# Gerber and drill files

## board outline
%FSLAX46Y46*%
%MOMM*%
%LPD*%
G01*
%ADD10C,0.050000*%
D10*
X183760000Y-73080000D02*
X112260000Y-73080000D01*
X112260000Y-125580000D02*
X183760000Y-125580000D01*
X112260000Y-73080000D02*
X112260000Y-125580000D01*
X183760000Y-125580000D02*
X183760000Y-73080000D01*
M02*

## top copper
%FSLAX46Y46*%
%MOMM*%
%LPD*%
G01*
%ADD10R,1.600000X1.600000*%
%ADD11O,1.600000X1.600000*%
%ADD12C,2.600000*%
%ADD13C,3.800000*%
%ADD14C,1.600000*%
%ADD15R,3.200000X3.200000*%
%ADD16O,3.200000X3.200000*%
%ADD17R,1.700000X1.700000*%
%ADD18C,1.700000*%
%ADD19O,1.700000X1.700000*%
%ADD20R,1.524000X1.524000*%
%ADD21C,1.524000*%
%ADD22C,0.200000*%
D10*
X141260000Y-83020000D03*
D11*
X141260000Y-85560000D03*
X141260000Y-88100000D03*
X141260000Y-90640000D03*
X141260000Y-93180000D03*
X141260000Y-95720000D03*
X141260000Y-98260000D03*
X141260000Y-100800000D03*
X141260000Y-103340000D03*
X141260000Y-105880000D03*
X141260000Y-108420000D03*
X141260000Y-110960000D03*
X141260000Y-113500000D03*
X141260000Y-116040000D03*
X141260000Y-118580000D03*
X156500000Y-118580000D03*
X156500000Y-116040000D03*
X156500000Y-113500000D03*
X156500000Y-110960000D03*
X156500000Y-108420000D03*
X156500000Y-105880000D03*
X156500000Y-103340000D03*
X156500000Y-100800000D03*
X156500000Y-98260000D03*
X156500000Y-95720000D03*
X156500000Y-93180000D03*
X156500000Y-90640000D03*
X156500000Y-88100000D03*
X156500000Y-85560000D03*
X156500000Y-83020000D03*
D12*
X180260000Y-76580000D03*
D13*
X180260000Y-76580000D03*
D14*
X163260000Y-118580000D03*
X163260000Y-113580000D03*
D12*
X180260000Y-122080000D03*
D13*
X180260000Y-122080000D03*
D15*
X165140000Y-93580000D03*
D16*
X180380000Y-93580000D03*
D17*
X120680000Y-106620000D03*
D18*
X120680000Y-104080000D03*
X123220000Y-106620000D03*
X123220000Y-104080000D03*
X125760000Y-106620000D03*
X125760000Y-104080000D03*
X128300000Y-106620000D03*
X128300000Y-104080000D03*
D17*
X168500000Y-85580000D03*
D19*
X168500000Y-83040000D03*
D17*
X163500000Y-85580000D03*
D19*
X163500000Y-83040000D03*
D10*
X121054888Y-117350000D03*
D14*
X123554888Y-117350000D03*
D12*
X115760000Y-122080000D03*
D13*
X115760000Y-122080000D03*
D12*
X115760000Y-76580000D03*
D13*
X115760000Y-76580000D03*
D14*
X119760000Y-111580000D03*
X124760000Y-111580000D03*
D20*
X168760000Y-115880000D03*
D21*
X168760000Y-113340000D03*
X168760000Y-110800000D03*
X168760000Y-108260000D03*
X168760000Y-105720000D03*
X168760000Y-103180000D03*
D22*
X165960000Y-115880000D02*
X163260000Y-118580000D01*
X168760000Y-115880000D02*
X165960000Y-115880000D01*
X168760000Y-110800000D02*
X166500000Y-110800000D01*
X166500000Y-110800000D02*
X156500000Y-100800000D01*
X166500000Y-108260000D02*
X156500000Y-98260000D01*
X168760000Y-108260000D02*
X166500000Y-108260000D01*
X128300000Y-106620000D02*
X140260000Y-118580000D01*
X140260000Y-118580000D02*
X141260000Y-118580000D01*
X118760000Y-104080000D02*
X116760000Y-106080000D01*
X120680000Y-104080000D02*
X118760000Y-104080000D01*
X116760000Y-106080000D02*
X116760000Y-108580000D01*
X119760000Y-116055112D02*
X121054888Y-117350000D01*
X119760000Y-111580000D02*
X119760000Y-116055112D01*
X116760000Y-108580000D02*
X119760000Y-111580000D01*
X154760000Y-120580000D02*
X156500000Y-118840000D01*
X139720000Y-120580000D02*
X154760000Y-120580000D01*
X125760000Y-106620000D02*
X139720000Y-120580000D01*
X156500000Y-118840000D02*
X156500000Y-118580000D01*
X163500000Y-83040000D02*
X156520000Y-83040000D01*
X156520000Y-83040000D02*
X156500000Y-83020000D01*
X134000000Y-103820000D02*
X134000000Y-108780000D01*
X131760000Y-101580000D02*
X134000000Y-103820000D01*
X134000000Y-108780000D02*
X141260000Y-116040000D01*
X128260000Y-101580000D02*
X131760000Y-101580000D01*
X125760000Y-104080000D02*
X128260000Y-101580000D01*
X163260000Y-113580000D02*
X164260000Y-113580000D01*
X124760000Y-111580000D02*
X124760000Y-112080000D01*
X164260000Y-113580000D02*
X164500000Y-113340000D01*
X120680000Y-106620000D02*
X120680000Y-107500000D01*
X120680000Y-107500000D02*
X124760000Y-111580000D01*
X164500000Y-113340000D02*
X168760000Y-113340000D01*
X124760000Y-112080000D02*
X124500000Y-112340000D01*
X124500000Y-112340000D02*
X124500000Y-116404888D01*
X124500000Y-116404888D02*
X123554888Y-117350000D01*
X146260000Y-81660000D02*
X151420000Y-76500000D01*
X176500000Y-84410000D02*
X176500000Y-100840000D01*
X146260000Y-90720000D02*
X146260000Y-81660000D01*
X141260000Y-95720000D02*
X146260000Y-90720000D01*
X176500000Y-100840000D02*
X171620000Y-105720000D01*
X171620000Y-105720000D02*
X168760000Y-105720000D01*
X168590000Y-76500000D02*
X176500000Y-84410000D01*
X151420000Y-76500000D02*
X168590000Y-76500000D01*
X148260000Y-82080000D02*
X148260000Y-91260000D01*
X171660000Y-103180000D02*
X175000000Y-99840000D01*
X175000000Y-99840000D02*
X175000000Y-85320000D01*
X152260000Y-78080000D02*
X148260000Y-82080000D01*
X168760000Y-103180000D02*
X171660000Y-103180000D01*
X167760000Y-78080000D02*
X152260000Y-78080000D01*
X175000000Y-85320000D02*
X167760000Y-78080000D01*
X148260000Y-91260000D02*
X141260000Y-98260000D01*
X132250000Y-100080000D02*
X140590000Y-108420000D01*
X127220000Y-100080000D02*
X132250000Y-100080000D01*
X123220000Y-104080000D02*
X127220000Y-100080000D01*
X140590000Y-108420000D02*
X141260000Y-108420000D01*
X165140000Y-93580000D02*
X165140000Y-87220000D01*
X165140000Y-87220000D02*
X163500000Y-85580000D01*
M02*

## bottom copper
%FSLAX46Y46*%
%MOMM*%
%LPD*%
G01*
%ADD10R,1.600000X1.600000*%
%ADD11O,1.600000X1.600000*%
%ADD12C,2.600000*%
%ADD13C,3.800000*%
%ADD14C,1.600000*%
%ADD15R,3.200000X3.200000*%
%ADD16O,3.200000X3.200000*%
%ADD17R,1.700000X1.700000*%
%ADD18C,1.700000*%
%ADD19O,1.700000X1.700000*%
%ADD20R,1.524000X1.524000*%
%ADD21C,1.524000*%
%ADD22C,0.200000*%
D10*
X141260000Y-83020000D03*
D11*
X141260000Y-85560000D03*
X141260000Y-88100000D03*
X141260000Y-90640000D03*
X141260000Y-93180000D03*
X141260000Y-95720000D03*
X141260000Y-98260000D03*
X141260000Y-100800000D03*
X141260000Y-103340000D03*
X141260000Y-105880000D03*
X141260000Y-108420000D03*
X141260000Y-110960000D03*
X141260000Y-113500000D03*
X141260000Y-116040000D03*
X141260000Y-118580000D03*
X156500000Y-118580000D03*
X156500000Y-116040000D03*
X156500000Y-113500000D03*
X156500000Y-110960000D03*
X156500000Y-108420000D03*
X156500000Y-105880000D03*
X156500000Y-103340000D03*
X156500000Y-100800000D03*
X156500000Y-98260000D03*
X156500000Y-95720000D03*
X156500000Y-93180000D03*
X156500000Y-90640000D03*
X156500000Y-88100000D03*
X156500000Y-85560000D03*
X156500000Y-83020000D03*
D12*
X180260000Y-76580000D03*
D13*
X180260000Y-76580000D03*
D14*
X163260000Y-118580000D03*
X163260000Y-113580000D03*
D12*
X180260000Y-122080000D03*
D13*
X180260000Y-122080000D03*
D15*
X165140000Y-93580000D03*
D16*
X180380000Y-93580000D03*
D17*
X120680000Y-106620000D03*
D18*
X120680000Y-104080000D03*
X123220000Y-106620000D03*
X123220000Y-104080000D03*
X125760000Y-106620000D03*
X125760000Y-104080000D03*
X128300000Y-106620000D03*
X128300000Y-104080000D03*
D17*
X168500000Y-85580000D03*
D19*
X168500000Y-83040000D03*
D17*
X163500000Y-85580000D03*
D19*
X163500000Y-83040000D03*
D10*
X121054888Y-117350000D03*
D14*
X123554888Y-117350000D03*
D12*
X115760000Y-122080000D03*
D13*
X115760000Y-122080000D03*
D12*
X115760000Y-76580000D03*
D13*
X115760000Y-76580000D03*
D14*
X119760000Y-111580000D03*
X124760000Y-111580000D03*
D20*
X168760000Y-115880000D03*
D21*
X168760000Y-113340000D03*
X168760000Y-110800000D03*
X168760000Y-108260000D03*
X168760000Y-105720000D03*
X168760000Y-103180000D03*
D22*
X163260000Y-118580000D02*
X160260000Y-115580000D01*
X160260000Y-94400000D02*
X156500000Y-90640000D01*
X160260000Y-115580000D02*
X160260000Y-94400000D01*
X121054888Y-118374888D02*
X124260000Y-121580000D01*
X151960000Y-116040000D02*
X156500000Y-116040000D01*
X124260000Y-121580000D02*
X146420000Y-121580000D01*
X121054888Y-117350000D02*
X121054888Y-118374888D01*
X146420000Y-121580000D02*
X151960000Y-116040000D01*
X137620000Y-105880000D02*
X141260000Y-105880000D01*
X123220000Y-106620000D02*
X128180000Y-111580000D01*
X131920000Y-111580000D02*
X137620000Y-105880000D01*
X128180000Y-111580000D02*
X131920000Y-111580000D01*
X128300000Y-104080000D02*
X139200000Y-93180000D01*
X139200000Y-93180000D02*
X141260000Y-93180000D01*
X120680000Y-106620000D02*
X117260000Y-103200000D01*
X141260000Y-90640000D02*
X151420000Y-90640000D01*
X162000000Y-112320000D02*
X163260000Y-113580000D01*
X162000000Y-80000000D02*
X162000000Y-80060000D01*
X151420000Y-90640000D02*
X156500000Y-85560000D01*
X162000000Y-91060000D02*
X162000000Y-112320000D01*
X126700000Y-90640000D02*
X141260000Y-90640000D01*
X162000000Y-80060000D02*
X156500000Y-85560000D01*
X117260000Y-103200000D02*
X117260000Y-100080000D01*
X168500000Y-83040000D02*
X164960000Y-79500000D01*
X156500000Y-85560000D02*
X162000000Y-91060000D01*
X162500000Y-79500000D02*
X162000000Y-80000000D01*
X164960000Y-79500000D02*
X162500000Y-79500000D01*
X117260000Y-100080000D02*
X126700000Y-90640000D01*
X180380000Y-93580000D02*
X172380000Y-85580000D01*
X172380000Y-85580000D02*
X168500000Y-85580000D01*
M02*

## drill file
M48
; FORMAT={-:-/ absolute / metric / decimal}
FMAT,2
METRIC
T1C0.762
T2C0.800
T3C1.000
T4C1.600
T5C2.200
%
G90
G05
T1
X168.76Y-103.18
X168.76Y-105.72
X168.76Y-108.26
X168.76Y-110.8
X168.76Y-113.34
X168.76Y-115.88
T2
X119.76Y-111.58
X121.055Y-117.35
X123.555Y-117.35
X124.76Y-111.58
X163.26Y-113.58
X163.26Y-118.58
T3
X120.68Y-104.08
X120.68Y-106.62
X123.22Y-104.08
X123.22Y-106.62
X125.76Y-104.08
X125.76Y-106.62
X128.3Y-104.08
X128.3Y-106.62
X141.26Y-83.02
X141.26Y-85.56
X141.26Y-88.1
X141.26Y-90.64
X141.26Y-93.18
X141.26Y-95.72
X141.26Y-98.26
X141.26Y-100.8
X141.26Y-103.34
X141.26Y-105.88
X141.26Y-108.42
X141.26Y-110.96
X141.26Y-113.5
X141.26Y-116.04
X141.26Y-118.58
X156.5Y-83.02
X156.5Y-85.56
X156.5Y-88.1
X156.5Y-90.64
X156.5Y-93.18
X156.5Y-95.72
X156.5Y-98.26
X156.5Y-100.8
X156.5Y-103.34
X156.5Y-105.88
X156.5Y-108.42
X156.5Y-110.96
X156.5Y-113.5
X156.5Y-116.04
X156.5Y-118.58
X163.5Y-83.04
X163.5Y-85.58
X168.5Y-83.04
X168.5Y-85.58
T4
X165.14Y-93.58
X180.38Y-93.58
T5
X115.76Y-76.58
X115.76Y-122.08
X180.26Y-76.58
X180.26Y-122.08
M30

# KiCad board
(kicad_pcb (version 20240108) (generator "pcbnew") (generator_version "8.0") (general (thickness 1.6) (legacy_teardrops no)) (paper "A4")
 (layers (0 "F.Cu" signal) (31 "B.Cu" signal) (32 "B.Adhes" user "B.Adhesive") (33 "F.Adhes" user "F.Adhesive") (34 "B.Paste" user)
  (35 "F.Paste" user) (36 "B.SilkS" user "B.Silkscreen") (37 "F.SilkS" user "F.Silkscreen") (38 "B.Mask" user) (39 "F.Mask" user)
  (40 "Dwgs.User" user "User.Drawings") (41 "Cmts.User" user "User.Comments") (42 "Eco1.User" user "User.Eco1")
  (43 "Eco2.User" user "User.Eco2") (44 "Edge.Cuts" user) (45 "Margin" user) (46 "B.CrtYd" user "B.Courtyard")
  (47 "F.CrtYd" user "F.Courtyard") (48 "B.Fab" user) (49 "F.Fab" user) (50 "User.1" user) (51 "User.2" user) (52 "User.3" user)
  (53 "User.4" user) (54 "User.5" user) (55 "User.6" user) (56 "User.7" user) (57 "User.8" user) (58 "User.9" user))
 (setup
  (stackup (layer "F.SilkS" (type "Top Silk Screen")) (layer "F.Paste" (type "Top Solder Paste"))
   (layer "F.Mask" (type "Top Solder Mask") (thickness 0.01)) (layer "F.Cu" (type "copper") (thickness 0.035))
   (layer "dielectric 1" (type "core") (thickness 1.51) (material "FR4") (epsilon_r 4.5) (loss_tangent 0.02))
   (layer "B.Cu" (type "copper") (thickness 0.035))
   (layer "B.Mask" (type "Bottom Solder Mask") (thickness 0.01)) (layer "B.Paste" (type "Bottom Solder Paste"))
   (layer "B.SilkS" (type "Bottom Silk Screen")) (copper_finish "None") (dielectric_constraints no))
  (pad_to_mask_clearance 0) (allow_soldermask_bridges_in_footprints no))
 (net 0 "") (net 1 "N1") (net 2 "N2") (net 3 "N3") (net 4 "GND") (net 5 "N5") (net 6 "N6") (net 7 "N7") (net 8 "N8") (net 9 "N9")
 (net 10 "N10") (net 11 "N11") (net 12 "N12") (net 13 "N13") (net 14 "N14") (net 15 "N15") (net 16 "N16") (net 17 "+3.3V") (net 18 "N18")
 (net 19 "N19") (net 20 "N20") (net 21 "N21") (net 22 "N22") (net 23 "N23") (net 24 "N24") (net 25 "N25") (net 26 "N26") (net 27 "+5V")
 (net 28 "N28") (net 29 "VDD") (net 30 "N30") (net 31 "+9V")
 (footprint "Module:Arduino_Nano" (layer "F.Cu") (at 141.26 83.02)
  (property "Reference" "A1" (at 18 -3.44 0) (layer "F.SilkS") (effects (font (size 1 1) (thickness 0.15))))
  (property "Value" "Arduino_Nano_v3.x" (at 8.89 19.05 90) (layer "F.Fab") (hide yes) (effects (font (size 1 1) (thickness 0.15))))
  (pad "1" thru_hole rect (at 0 0) (size 1.6 1.6) (drill 1) (layers "*.Cu" "*.Mask") (remove_unused_layers no) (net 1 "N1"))
  (pad "2" thru_hole oval (at 0 2.54) (size 1.6 1.6) (drill 1) (layers "*.Cu" "*.Mask") (remove_unused_layers no) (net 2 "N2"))
  (pad "3" thru_hole oval (at 0 5.08) (size 1.6 1.6) (drill 1) (layers "*.Cu" "*.Mask") (remove_unused_layers no) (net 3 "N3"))
  (pad "4" thru_hole oval (at 0 7.62) (size 1.6 1.6) (drill 1) (layers "*.Cu" "*.Mask") (remove_unused_layers no) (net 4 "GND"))
  (pad "5" thru_hole oval (at 0 10.16) (size 1.6 1.6) (drill 1) (layers "*.Cu" "*.Mask") (remove_unused_layers no) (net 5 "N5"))
  (pad "6" thru_hole oval (at 0 12.7) (size 1.6 1.6) (drill 1) (layers "*.Cu" "*.Mask") (remove_unused_layers no) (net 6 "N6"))
  (pad "7" thru_hole oval (at 0 15.24) (size 1.6 1.6) (drill 1) (layers "*.Cu" "*.Mask") (remove_unused_layers no) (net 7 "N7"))
  (pad "8" thru_hole oval (at 0 17.78) (size 1.6 1.6) (drill 1) (layers "*.Cu" "*.Mask") (remove_unused_layers no) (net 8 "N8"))
  (pad "9" thru_hole oval (at 0 20.32) (size 1.6 1.6) (drill 1) (layers "*.Cu" "*.Mask") (remove_unused_layers no) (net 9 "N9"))
  (pad "10" thru_hole oval (at 0 22.86) (size 1.6 1.6) (drill 1) (layers "*.Cu" "*.Mask") (remove_unused_layers no) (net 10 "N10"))
  (pad "11" thru_hole oval (at 0 25.4) (size 1.6 1.6) (drill 1) (layers "*.Cu" "*.Mask") (remove_unused_layers no) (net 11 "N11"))
  (pad "12" thru_hole oval (at 0 27.94) (size 1.6 1.6) (drill 1) (layers "*.Cu" "*.Mask") (remove_unused_layers no) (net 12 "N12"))
  (pad "13" thru_hole oval (at 0 30.48) (size 1.6 1.6) (drill 1) (layers "*.Cu" "*.Mask") (remove_unused_layers no) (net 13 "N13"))
  (pad "14" thru_hole oval (at 0 33.02) (size 1.6 1.6) (drill 1) (layers "*.Cu" "*.Mask") (remove_unused_layers no) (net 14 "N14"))
  (pad "15" thru_hole oval (at 0 35.56) (size 1.6 1.6) (drill 1) (layers "*.Cu" "*.Mask") (remove_unused_layers no) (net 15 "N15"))
  (pad "16" thru_hole oval (at 15.24 35.56) (size 1.6 1.6) (drill 1) (layers "*.Cu" "*.Mask") (remove_unused_layers no) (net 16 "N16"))
  (pad "17" thru_hole oval (at 15.24 33.02) (size 1.6 1.6) (drill 1) (layers "*.Cu" "*.Mask") (remove_unused_layers no) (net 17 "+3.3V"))
  (pad "18" thru_hole oval (at 15.24 30.48) (size 1.6 1.6) (drill 1) (layers "*.Cu" "*.Mask") (remove_unused_layers no) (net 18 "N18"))
  (pad "19" thru_hole oval (at 15.24 27.94) (size 1.6 1.6) (drill 1) (layers "*.Cu" "*.Mask") (remove_unused_layers no) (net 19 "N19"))
  (pad "20" thru_hole oval (at 15.24 25.4) (size 1.6 1.6) (drill 1) (layers "*.Cu" "*.Mask") (remove_unused_layers no) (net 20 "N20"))
  (pad "21" thru_hole oval (at 15.24 22.86) (size 1.6 1.6) (drill 1) (layers "*.Cu" "*.Mask") (remove_unused_layers no) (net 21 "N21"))
  (pad "22" thru_hole oval (at 15.24 20.32) (size 1.6 1.6) (drill 1) (layers "*.Cu" "*.Mask") (remove_unused_layers no) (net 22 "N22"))
  (pad "23" thru_hole oval (at 15.24 17.78) (size 1.6 1.6) (drill 1) (layers "*.Cu" "*.Mask") (remove_unused_layers no) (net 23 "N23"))
  (pad "24" thru_hole oval (at 15.24 15.24) (size 1.6 1.6) (drill 1) (layers "*.Cu" "*.Mask") (remove_unused_layers no) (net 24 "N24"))
  (pad "25" thru_hole oval (at 15.24 12.7) (size 1.6 1.6) (drill 1) (layers "*.Cu" "*.Mask") (remove_unused_layers no) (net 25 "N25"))
  (pad "26" thru_hole oval (at 15.24 10.16) (size 1.6 1.6) (drill 1) (layers "*.Cu" "*.Mask") (remove_unused_layers no) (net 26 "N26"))
  (pad "27" thru_hole oval (at 15.24 7.62) (size 1.6 1.6) (drill 1) (layers "*.Cu" "*.Mask") (remove_unused_layers no) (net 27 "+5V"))
  (pad "28" thru_hole oval (at 15.24 5.08) (size 1.6 1.6) (drill 1) (layers "*.Cu" "*.Mask") (remove_unused_layers no) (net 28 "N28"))
  (pad "29" thru_hole oval (at 15.24 2.54) (size 1.6 1.6) (drill 1) (layers "*.Cu" "*.Mask") (remove_unused_layers no) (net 4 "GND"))
  (pad "30" thru_hole oval (at 15.24 0) (size 1.6 1.6) (drill 1) (layers "*.Cu" "*.Mask") (remove_unused_layers no) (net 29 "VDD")))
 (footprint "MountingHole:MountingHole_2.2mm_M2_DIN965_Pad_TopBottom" (layer "F.Cu") (at 180.26 76.58)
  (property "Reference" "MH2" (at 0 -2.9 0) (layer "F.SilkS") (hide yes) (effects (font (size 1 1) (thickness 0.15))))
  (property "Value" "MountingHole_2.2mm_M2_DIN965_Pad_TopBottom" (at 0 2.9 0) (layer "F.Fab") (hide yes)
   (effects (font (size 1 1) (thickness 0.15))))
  (pad "1" thru_hole circle (at 0 0) (size 2.6 2.6) (drill 2.2) (layers "*.Cu" "*.Mask") (remove_unused_layers no))
  (pad "1" connect circle (at 0 0) (size 3.8 3.8) (layers "F.Cu" "F.Mask"))
  (pad "1" connect circle (at 0 0) (size 3.8 3.8) (layers "B.Cu" "B.Mask")))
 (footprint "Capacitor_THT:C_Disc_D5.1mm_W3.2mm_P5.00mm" (layer "F.Cu") (at 163.26 118.58 90)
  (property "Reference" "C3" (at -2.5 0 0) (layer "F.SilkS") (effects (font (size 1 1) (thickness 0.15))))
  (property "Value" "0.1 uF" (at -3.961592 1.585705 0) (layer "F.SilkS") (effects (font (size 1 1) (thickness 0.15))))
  (pad "1" thru_hole circle (at 0 0 90) (size 1.6 1.6) (drill 0.8) (layers "*.Cu" "*.Mask") (remove_unused_layers no) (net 27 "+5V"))
  (pad "2" thru_hole circle (at 5 0 90) (size 1.6 1.6) (drill 0.8) (layers "*.Cu" "*.Mask") (remove_unused_layers no) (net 4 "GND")))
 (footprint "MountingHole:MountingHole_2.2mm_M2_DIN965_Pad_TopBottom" (layer "F.Cu") (at 180.26 122.08)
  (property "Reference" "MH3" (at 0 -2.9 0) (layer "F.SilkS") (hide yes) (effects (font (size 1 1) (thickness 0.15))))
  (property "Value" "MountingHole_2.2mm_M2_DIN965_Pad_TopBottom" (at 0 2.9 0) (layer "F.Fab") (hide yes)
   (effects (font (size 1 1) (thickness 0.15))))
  (pad "1" thru_hole circle (at 0 0) (size 2.6 2.6) (drill 2.2) (layers "*.Cu" "*.Mask") (remove_unused_layers no))
  (pad "1" connect circle (at 0 0) (size 3.8 3.8) (layers "F.Cu" "F.Mask"))
  (pad "1" connect circle (at 0 0) (size 3.8 3.8) (layers "B.Cu" "B.Mask")))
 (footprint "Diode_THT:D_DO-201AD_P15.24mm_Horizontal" (layer "F.Cu") (at 165.14 93.58)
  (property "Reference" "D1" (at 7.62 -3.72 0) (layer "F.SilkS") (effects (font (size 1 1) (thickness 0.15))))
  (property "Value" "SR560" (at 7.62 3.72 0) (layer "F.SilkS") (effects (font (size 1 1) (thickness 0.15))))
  (pad "1" thru_hole rect (at 0 0) (size 3.2 3.2) (drill 1.6) (layers "*.Cu" "*.Mask") (remove_unused_layers no) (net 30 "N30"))
  (pad "2" thru_hole oval (at 15.24 0) (size 3.2 3.2) (drill 1.6) (layers "*.Cu" "*.Mask") (remove_unused_layers no) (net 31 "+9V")))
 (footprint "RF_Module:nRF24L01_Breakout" (layer "F.Cu") (at 120.68 106.62 90)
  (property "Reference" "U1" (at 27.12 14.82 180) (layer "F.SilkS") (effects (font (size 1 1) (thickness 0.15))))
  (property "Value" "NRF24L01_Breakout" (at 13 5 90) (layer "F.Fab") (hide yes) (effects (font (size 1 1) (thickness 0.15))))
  (pad "1" thru_hole rect (at 0 0 90) (size 1.7 1.7) (drill 1) (layers "*.Cu" "*.Mask") (remove_unused_layers no) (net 4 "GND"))
  (pad "2" thru_hole circle (at 2.54 0 90) (size 1.7 1.7) (drill 1) (layers "*.Cu" "*.Mask") (remove_unused_layers no) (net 17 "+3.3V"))
  (pad "3" thru_hole circle (at 0 2.54 90) (size 1.7 1.7) (drill 1) (layers "*.Cu" "*.Mask") (remove_unused_layers no) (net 10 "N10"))
  (pad "4" thru_hole circle (at 2.54 2.54 90) (size 1.7 1.7) (drill 1) (layers "*.Cu" "*.Mask") (remove_unused_layers no) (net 11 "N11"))
  (pad "5" thru_hole circle (at 0 5.08 90) (size 1.7 1.7) (drill 1) (layers "*.Cu" "*.Mask") (remove_unused_layers no) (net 16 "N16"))
  (pad "6" thru_hole circle (at 2.54 5.08 90) (size 1.7 1.7) (drill 1) (layers "*.Cu" "*.Mask") (remove_unused_layers no) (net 14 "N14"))
  (pad "7" thru_hole circle (at 0 7.62 90) (size 1.7 1.7) (drill 1) (layers "*.Cu" "*.Mask") (remove_unused_layers no) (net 15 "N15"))
  (pad "8" thru_hole circle (at 2.54 7.62 90) (size 1.7 1.7) (drill 1) (layers "*.Cu" "*.Mask") (remove_unused_layers no) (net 5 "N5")))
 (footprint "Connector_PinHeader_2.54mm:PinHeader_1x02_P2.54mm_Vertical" (layer "F.Cu") (at 168.5 85.58 180)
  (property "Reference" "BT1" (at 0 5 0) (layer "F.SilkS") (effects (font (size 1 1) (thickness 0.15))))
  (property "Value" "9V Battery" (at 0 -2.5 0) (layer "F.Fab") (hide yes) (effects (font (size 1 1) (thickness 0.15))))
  (pad "1" thru_hole rect (at 0 0 180) (size 1.7 1.7) (drill 1) (layers "*.Cu" "*.Mask") (remove_unused_layers no) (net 31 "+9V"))
  (pad "2" thru_hole oval (at 0 2.54 180) (size 1.7 1.7) (drill 1) (layers "*.Cu" "*.Mask") (remove_unused_layers no) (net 4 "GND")))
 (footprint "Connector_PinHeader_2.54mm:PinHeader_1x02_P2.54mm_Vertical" (layer "F.Cu") (at 163.5 85.58 180)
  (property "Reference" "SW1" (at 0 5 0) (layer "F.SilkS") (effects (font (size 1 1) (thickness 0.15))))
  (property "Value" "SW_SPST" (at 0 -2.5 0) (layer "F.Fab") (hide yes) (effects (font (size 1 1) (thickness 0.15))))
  (pad "1" thru_hole rect (at 0 0 180) (size 1.7 1.7) (drill 1) (layers "*.Cu" "*.Mask") (remove_unused_layers no) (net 30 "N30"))
  (pad "2" thru_hole oval (at 0 2.54 180) (size 1.7 1.7) (drill 1) (layers "*.Cu" "*.Mask") (remove_unused_layers no) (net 29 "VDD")))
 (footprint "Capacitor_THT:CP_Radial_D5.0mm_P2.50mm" (layer "F.Cu") (at 121.054888 117.35)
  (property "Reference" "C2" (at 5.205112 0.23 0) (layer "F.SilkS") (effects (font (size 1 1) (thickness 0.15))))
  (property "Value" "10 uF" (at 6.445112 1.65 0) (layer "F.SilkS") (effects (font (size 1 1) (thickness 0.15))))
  (pad "1" thru_hole rect (at 0 0) (size 1.6 1.6) (drill 0.8) (layers "*.Cu" "*.Mask") (remove_unused_layers no) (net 17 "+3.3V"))
  (pad "2" thru_hole circle (at 2.5 0) (size 1.6 1.6) (drill 0.8) (layers "*.Cu" "*.Mask") (remove_unused_layers no) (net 4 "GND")))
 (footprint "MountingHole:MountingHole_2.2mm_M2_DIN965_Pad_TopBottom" (layer "F.Cu") (at 115.76 122.08)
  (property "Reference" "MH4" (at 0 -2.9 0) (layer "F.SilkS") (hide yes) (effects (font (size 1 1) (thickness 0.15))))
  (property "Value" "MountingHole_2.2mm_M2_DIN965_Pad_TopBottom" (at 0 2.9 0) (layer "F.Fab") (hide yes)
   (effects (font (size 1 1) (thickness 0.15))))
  (pad "1" thru_hole circle (at 0 0) (size 2.6 2.6) (drill 2.2) (layers "*.Cu" "*.Mask") (remove_unused_layers no))
  (pad "1" connect circle (at 0 0) (size 3.8 3.8) (layers "F.Cu" "F.Mask"))
  (pad "1" connect circle (at 0 0) (size 3.8 3.8) (layers "B.Cu" "B.Mask")))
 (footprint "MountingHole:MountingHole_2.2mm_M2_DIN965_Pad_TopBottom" (layer "F.Cu") (at 115.76 76.58)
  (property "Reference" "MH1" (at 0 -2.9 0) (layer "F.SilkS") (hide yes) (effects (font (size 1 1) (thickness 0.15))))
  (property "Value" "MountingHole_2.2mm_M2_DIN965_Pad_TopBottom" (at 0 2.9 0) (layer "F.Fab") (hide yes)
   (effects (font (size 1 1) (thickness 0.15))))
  (pad "1" thru_hole circle (at 0 0) (size 2.6 2.6) (drill 2.2) (layers "*.Cu" "*.Mask") (remove_unused_layers no))
  (pad "1" connect circle (at 0 0) (size 3.8 3.8) (layers "F.Cu" "F.Mask"))
  (pad "1" connect circle (at 0 0) (size 3.8 3.8) (layers "B.Cu" "B.Mask")))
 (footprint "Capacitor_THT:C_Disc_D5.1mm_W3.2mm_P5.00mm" (layer "F.Cu") (at 119.76 111.58)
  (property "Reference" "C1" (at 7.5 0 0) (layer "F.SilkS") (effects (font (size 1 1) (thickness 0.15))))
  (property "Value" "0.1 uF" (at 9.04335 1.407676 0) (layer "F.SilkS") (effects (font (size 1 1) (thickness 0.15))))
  (pad "1" thru_hole circle (at 0 0) (size 1.6 1.6) (drill 0.8) (layers "*.Cu" "*.Mask") (remove_unused_layers no) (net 17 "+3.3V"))
  (pad "2" thru_hole circle (at 5 0) (size 1.6 1.6) (drill 0.8) (layers "*.Cu" "*.Mask") (remove_unused_layers no) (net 4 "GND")))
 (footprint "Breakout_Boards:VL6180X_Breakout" (layer "F.Cu") (at 173.26 109.58 -90)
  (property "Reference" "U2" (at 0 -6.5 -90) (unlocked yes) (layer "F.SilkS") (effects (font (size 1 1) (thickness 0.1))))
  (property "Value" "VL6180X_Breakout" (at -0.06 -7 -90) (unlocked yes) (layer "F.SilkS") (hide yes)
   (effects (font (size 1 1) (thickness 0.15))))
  (pad "1" thru_hole rect (at 6.3 4.5 270) (size 1.524 1.524) (drill 0.762) (layers "*.Cu" "*.Mask") (remove_unused_layers no)
   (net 27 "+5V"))
  (pad "2" thru_hole circle (at 3.76 4.5 270) (size 1.524 1.524) (drill 0.762) (layers "*.Cu" "*.Mask") (remove_unused_layers no)
   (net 4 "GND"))
  (pad "3" thru_hole circle (at 1.22 4.5 270) (size 1.524 1.524) (drill 0.762) (layers "*.Cu" "*.Mask") (remove_unused_layers no)
   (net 23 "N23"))
  (pad "4" thru_hole circle (at -1.32 4.5 270) (size 1.524 1.524) (drill 0.762) (layers "*.Cu" "*.Mask") (remove_unused_layers no)
   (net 24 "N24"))
  (pad "5" thru_hole circle (at -3.86 4.5 270) (size 1.524 1.524) (drill 0.762) (layers "*.Cu" "*.Mask") (remove_unused_layers no)
   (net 6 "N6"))
  (pad "6" thru_hole circle (at -6.4 4.5 270) (size 1.524 1.524) (drill 0.762) (layers "*.Cu" "*.Mask") (remove_unused_layers no)
   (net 7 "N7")))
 (gr_line (start 183.76 73.08) (end 112.26 73.08) (stroke (width 0.05) (type default)) (layer "Edge.Cuts"))
 (gr_line (start 112.26 125.58) (end 183.76 125.58) (stroke (width 0.05) (type default)) (layer "Edge.Cuts"))
 (gr_line (start 112.26 73.08) (end 112.26 125.58) (stroke (width 0.05) (type default)) (layer "Edge.Cuts"))
 (gr_line (start 183.76 125.58) (end 183.76 73.08) (stroke (width 0.05) (type default)) (layer "Edge.Cuts"))
 (segment (start 165.96 115.88) (end 163.26 118.58) (width 0.2) (layer "F.Cu") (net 27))
 (segment (start 168.76 115.88) (end 165.96 115.88) (width 0.2) (layer "F.Cu") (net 27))
 (segment (start 163.26 118.58) (end 160.26 115.58) (width 0.2) (layer "B.Cu") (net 27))
 (segment (start 160.26 94.4) (end 156.5 90.64) (width 0.2) (layer "B.Cu") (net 27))
 (segment (start 160.26 115.58) (end 160.26 94.4) (width 0.2) (layer "B.Cu") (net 27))
 (segment (start 168.76 110.8) (end 166.5 110.8) (width 0.2) (layer "F.Cu") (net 23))
 (segment (start 166.5 110.8) (end 156.5 100.8) (width 0.2) (layer "F.Cu") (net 23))
 (segment (start 166.5 108.26) (end 156.5 98.26) (width 0.2) (layer "F.Cu") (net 24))
 (segment (start 168.76 108.26) (end 166.5 108.26) (width 0.2) (layer "F.Cu") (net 24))
 (segment (start 128.3 106.62) (end 140.26 118.58) (width 0.2) (layer "F.Cu") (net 15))
 (segment (start 140.26 118.58) (end 141.26 118.58) (width 0.2) (layer "F.Cu") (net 15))
 (segment (start 118.76 104.08) (end 116.76 106.08) (width 0.2) (layer "F.Cu") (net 17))
 (segment (start 120.68 104.08) (end 118.76 104.08) (width 0.2) (layer "F.Cu") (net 17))
 (segment (start 116.76 106.08) (end 116.76 108.58) (width 0.2) (layer "F.Cu") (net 17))
 (segment (start 119.76 116.055112) (end 121.054888 117.35) (width 0.2) (layer "F.Cu") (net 17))
 (segment (start 119.76 111.58) (end 119.76 116.055112) (width 0.2) (layer "F.Cu") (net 17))
 (segment (start 116.76 108.58) (end 119.76 111.58) (width 0.2) (layer "F.Cu") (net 17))
 (segment (start 121.054888 118.374888) (end 124.26 121.58) (width 0.2) (layer "B.Cu") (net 17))
 (segment (start 151.96 116.04) (end 156.5 116.04) (width 0.2) (layer "B.Cu") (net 17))
 (segment (start 124.26 121.58) (end 146.42 121.58) (width 0.2) (layer "B.Cu") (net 17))
 (segment (start 121.054888 117.35) (end 121.054888 118.374888) (width 0.2) (layer "B.Cu") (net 17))
 (segment (start 146.42 121.58) (end 151.96 116.04) (width 0.2) (layer "B.Cu") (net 17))
 (segment (start 137.62 105.88) (end 141.26 105.88) (width 0.2) (layer "B.Cu") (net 10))
 (segment (start 123.22 106.62) (end 128.18 111.58) (width 0.2) (layer "B.Cu") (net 10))
 (segment (start 131.92 111.58) (end 137.62 105.88) (width 0.2) (layer "B.Cu") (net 10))
 (segment (start 128.18 111.58) (end 131.92 111.58) (width 0.2) (layer "B.Cu") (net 10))
 (segment (start 154.76 120.58) (end 156.5 118.84) (width 0.2) (layer "F.Cu") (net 16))
 (segment (start 139.72 120.58) (end 154.76 120.58) (width 0.2) (layer "F.Cu") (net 16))
 (segment (start 125.76 106.62) (end 139.72 120.58) (width 0.2) (layer "F.Cu") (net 16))
 (segment (start 156.5 118.84) (end 156.5 118.58) (width 0.2) (layer "F.Cu") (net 16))
 (segment (start 163.5 83.04) (end 156.52 83.04) (width 0.2) (layer "F.Cu") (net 29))
 (segment (start 156.52 83.04) (end 156.5 83.02) (width 0.2) (layer "F.Cu") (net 29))
 (segment (start 128.3 104.08) (end 139.2 93.18) (width 0.2) (layer "B.Cu") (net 5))
 (segment (start 139.2 93.18) (end 141.26 93.18) (width 0.2) (layer "B.Cu") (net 5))
 (segment (start 134 103.82) (end 134 108.78) (width 0.2) (layer "F.Cu") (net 14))
 (segment (start 131.76 101.58) (end 134 103.82) (width 0.2) (layer "F.Cu") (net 14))
 (segment (start 134 108.78) (end 141.26 116.04) (width 0.2) (layer "F.Cu") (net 14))
 (segment (start 128.26 101.58) (end 131.76 101.58) (width 0.2) (layer "F.Cu") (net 14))
 (segment (start 125.76 104.08) (end 128.26 101.58) (width 0.2) (layer "F.Cu") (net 14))
 (segment (start 163.26 113.58) (end 164.26 113.58) (width 0.2) (layer "F.Cu") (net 4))
 (segment (start 124.76 111.58) (end 124.76 112.08) (width 0.2) (layer "F.Cu") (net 4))
 (segment (start 164.26 113.58) (end 164.5 113.34) (width 0.2) (layer "F.Cu") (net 4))
 (segment (start 120.68 106.62) (end 120.68 107.5) (width 0.2) (layer "F.Cu") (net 4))
 (segment (start 120.68 107.5) (end 124.76 111.58) (width 0.2) (layer "F.Cu") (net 4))
 (segment (start 164.5 113.34) (end 168.76 113.34) (width 0.2) (layer "F.Cu") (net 4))
 (segment (start 124.76 112.08) (end 124.5 112.34) (width 0.2) (layer "F.Cu") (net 4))
 (segment (start 124.5 112.34) (end 124.5 116.404888) (width 0.2) (layer "F.Cu") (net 4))
 (segment (start 124.5 116.404888) (end 123.554888 117.35) (width 0.2) (layer "F.Cu") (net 4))
 (segment (start 120.68 106.62) (end 117.26 103.2) (width 0.2) (layer "B.Cu") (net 4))
 (segment (start 141.26 90.64) (end 151.42 90.64) (width 0.2) (layer "B.Cu") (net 4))
 (segment (start 162 112.32) (end 163.26 113.58) (width 0.2) (layer "B.Cu") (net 4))
 (segment (start 162 80) (end 162 80.06) (width 0.2) (layer "B.Cu") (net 4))
 (segment (start 151.42 90.64) (end 156.5 85.56) (width 0.2) (layer "B.Cu") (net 4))
 (segment (start 162 91.06) (end 162 112.32) (width 0.2) (layer "B.Cu") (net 4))
 (segment (start 126.7 90.64) (end 141.26 90.64) (width 0.2) (layer "B.Cu") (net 4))
 (segment (start 162 80.06) (end 156.5 85.56) (width 0.2) (layer "B.Cu") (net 4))
 (segment (start 117.26 103.2) (end 117.26 100.08) (width 0.2) (layer "B.Cu") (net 4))
 (segment (start 168.5 83.04) (end 164.96 79.5) (width 0.2) (layer "B.Cu") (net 4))
 (segment (start 156.5 85.56) (end 162 91.06) (width 0.2) (layer "B.Cu") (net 4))
 (segment (start 162.5 79.5) (end 162 80) (width 0.2) (layer "B.Cu") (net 4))
 (segment (start 164.96 79.5) (end 162.5 79.5) (width 0.2) (layer "B.Cu") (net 4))
 (segment (start 117.26 100.08) (end 126.7 90.64) (width 0.2) (layer "B.Cu") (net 4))
 (segment (start 146.26 81.66) (end 151.42 76.5) (width 0.2) (layer "F.Cu") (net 6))
 (segment (start 176.5 84.41) (end 176.5 100.84) (width 0.2) (layer "F.Cu") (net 6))
 (segment (start 146.26 90.72) (end 146.26 81.66) (width 0.2) (layer "F.Cu") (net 6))
 (segment (start 141.26 95.72) (end 146.26 90.72) (width 0.2) (layer "F.Cu") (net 6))
 (segment (start 176.5 100.84) (end 171.62 105.72) (width 0.2) (layer "F.Cu") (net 6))
 (segment (start 171.62 105.72) (end 168.76 105.72) (width 0.2) (layer "F.Cu") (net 6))
 (segment (start 168.59 76.5) (end 176.5 84.41) (width 0.2) (layer "F.Cu") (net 6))
 (segment (start 151.42 76.5) (end 168.59 76.5) (width 0.2) (layer "F.Cu") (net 6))
 (segment (start 148.26 82.08) (end 148.26 91.26) (width 0.2) (layer "F.Cu") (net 7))
 (segment (start 171.66 103.18) (end 175 99.84) (width 0.2) (layer "F.Cu") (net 7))
 (segment (start 175 99.84) (end 175 85.32) (width 0.2) (layer "F.Cu") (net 7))
 (segment (start 152.26 78.08) (end 148.26 82.08) (width 0.2) (layer "F.Cu") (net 7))
 (segment (start 168.76 103.18) (end 171.66 103.18) (width 0.2) (layer "F.Cu") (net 7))
 (segment (start 167.76 78.08) (end 152.26 78.08) (width 0.2) (layer "F.Cu") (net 7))
 (segment (start 175 85.32) (end 167.76 78.08) (width 0.2) (layer "F.Cu") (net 7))
 (segment (start 148.26 91.26) (end 141.26 98.26) (width 0.2) (layer "F.Cu") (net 7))
 (segment (start 132.25 100.08) (end 140.59 108.42) (width 0.2) (layer "F.Cu") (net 11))
 (segment (start 127.22 100.08) (end 132.25 100.08) (width 0.2) (layer "F.Cu") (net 11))
 (segment (start 123.22 104.08) (end 127.22 100.08) (width 0.2) (layer "F.Cu") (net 11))
 (segment (start 140.59 108.42) (end 141.26 108.42) (width 0.2) (layer "F.Cu") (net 11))
 (segment (start 180.38 93.58) (end 172.38 85.58) (width 0.2) (layer "B.Cu") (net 31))
 (segment (start 172.38 85.58) (end 168.5 85.58) (width 0.2) (layer "B.Cu") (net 31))
 (segment (start 165.14 93.58) (end 165.14 87.22) (width 0.2) (layer "F.Cu") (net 30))
 (segment (start 165.14 87.22) (end 163.5 85.58) (width 0.2) (layer "F.Cu") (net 30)))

